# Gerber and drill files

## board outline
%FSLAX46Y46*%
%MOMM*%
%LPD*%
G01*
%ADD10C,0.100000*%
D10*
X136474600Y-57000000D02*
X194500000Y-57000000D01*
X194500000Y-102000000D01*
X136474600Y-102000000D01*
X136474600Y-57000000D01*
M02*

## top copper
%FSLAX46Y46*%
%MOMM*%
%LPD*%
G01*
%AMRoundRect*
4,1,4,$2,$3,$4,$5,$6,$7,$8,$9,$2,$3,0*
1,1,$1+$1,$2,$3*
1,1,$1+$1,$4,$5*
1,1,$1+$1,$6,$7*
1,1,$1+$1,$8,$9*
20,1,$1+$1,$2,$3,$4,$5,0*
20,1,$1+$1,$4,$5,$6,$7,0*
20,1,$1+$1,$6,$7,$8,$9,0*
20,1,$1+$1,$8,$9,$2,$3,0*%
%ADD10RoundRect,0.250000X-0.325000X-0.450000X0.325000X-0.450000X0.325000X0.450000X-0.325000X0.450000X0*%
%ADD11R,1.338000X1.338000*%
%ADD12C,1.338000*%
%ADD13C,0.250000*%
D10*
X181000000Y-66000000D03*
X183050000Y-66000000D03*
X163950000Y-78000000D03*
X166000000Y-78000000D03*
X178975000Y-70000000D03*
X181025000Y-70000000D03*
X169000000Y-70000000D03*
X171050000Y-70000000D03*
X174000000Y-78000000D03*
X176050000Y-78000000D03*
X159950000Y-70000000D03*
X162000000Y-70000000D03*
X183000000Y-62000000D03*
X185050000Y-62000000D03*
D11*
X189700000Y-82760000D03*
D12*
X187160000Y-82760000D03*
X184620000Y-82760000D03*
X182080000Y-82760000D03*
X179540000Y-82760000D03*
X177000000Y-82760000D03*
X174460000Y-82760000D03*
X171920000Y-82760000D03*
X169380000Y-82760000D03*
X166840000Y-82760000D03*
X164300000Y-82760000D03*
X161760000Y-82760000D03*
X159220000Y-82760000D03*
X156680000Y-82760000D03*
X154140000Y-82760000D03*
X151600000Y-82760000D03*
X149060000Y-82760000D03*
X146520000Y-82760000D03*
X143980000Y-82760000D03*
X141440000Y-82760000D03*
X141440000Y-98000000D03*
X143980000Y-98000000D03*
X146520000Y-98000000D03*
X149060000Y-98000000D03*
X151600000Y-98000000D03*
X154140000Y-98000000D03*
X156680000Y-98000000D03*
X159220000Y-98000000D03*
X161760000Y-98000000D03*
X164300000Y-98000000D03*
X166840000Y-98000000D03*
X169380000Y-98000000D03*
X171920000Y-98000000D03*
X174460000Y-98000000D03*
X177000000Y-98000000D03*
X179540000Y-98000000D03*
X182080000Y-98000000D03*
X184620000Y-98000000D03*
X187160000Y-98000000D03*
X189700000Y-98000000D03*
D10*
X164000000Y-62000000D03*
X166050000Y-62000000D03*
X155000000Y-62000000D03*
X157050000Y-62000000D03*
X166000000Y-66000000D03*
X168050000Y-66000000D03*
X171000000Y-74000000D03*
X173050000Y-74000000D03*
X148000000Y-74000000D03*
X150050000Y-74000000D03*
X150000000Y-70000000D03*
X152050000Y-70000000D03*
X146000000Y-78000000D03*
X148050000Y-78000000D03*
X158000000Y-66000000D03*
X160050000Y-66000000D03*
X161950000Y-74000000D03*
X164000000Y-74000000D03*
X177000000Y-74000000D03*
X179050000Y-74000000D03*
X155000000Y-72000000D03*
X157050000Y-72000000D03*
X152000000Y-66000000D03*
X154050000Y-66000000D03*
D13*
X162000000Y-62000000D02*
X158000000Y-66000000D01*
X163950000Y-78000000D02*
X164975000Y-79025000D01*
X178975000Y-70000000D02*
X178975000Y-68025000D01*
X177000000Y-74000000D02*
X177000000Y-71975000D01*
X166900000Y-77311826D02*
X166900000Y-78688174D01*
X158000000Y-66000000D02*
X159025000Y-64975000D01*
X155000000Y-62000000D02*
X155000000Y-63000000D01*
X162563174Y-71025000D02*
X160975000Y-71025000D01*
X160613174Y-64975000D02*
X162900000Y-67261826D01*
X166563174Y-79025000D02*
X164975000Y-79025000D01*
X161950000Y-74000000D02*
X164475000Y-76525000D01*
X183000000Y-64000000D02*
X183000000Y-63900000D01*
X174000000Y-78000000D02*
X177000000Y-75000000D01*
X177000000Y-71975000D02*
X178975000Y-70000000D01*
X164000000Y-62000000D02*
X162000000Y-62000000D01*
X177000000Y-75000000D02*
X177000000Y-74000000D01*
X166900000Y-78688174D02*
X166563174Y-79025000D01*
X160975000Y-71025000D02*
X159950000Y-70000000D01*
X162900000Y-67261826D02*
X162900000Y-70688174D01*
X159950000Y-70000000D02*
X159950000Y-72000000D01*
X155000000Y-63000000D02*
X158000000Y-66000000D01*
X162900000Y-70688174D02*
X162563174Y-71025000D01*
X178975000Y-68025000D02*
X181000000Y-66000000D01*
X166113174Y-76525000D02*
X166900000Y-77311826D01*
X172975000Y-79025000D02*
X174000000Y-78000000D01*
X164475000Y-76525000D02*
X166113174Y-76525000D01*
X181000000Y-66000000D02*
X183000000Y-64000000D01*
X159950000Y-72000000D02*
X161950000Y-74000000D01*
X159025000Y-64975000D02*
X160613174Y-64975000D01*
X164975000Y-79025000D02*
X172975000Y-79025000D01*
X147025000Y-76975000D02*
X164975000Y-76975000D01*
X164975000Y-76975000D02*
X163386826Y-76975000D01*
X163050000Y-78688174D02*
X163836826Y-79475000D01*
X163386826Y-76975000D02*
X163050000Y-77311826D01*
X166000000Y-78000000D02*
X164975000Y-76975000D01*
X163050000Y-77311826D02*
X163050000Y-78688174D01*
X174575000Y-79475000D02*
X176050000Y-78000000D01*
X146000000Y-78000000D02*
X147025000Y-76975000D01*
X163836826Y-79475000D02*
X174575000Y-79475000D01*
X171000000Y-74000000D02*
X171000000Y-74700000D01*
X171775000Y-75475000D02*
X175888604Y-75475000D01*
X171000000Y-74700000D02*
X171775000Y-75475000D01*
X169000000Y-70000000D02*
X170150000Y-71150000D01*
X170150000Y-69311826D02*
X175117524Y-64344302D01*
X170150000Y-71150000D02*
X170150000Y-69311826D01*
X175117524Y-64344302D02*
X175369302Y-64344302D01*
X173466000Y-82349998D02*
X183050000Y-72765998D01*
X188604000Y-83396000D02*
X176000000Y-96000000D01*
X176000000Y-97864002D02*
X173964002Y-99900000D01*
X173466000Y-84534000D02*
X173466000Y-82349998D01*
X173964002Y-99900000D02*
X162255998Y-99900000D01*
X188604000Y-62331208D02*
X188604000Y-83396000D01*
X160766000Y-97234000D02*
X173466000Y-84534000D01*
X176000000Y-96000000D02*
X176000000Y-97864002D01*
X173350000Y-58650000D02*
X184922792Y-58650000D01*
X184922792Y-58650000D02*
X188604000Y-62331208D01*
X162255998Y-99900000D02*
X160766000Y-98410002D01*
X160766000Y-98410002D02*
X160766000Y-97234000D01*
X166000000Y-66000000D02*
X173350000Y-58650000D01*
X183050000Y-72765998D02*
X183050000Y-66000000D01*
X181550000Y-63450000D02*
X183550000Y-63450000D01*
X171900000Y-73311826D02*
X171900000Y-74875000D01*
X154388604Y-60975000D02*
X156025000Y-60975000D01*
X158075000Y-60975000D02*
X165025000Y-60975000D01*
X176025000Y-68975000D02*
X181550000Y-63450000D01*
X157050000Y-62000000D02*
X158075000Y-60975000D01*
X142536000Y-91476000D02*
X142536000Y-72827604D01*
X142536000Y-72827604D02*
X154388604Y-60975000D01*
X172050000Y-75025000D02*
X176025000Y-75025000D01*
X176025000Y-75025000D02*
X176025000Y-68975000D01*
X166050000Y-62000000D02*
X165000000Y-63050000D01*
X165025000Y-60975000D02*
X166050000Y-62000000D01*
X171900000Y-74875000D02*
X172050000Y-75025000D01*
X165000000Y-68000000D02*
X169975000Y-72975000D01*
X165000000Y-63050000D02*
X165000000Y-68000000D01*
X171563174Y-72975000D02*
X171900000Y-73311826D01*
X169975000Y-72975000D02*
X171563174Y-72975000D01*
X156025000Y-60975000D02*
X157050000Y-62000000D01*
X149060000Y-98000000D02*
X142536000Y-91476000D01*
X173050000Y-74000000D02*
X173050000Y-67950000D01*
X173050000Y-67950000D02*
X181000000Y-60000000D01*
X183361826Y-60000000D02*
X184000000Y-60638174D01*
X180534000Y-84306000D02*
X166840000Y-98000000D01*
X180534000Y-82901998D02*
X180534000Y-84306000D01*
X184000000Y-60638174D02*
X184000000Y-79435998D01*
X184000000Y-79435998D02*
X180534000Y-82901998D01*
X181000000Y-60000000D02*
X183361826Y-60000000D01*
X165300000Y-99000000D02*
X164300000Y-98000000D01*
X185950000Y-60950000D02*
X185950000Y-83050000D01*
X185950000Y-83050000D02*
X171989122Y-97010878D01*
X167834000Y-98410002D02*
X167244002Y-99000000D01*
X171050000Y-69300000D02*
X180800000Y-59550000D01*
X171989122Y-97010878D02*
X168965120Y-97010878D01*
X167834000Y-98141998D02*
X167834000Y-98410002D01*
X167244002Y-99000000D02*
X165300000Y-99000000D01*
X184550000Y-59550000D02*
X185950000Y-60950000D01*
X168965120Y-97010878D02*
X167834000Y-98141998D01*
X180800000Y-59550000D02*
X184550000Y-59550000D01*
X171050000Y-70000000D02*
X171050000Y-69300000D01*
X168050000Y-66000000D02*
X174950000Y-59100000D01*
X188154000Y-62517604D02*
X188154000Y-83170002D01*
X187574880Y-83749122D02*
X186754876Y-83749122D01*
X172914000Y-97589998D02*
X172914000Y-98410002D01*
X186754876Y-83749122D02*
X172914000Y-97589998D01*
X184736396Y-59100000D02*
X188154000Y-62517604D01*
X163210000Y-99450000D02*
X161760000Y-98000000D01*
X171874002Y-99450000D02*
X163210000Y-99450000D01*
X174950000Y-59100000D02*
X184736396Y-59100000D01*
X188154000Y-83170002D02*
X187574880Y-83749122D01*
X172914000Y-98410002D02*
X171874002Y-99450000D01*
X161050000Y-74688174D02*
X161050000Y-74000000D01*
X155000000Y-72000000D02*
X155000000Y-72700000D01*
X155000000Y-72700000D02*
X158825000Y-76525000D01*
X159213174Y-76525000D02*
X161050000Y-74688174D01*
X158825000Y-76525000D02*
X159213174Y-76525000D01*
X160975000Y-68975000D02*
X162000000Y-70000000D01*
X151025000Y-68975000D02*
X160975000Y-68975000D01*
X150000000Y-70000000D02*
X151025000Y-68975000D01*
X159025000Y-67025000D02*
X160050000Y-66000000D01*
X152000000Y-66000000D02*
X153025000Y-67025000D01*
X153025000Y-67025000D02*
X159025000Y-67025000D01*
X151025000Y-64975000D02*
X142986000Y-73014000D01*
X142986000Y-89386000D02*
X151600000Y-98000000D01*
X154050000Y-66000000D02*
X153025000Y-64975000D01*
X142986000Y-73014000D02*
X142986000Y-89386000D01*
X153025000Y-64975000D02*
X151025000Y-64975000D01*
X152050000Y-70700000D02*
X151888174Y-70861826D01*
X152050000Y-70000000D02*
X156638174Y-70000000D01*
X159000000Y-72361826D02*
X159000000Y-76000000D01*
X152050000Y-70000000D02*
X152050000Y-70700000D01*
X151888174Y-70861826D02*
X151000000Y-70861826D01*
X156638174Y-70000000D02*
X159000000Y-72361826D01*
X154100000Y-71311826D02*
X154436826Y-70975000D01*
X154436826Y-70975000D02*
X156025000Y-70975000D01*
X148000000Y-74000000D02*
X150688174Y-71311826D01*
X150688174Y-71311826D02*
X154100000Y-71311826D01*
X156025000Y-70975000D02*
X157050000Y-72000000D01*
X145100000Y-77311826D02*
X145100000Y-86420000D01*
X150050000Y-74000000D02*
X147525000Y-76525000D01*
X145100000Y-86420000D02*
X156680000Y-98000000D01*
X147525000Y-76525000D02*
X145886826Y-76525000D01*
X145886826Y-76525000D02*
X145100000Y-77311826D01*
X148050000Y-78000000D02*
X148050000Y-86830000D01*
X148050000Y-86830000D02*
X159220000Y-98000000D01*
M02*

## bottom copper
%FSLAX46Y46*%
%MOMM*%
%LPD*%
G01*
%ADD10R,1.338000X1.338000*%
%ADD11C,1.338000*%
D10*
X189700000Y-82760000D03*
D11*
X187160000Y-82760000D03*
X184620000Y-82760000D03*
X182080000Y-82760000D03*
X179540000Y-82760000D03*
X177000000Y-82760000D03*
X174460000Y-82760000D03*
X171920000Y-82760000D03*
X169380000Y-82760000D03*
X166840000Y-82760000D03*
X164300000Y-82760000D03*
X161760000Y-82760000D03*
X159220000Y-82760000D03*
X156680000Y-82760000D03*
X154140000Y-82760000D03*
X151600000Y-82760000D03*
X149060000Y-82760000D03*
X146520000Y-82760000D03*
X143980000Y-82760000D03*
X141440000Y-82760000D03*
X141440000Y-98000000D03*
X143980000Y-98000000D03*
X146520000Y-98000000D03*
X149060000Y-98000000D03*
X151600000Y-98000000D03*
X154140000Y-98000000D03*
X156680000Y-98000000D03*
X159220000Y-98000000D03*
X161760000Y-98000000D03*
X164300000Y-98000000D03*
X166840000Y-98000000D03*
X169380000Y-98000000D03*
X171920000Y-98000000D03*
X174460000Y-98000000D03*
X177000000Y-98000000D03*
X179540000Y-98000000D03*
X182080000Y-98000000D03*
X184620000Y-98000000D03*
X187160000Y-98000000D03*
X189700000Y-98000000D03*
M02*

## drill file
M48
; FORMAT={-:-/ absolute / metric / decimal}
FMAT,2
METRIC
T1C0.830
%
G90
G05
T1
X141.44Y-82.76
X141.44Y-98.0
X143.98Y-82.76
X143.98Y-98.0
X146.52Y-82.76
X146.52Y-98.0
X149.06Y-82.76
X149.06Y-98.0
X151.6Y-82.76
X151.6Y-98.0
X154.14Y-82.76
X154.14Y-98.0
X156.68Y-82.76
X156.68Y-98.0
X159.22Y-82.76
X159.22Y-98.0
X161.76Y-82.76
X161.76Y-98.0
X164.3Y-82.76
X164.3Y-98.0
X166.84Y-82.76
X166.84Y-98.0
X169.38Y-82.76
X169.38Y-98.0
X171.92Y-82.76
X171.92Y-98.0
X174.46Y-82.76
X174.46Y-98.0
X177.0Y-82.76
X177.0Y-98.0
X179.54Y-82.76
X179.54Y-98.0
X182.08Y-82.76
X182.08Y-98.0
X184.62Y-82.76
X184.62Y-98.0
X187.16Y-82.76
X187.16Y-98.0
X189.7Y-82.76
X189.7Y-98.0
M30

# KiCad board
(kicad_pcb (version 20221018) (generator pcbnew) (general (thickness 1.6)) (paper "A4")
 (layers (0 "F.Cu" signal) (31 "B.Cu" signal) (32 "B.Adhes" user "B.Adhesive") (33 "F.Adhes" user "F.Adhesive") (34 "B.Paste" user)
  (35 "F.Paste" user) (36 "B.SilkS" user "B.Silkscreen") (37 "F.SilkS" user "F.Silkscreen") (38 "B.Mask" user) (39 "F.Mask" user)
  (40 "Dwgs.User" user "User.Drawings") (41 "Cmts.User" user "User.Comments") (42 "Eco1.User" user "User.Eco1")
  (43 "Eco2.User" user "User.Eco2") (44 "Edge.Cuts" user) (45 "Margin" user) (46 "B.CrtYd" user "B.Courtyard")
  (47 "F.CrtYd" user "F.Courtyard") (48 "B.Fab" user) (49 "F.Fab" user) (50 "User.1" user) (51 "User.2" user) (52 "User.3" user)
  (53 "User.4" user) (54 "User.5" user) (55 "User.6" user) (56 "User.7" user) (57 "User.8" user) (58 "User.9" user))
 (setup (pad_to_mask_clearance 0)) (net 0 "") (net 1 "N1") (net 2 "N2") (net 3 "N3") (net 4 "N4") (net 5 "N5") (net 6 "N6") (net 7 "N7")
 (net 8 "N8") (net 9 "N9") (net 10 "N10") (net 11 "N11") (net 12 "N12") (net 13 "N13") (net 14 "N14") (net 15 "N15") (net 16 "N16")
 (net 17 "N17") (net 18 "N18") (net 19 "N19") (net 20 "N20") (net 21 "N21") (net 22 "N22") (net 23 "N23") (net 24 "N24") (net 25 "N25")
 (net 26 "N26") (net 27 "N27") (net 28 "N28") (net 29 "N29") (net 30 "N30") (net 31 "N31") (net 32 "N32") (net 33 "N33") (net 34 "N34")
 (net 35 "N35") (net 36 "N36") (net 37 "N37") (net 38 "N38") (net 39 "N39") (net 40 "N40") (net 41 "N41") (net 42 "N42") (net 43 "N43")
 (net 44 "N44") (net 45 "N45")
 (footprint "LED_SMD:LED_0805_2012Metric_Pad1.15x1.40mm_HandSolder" (layer "F.Cu") (at 182.025 66)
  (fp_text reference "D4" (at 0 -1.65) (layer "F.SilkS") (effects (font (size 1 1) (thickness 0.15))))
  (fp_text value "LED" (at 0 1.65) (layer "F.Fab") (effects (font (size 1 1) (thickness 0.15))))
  (pad "1" smd roundrect (at -1.025 0) (size 1.15 1.4) (layers "F.Cu" "F.Paste" "F.Mask") (roundrect_rratio 0.217391) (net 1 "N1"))
  (pad "2" smd roundrect (at 1.025 0) (size 1.15 1.4) (layers "F.Cu" "F.Paste" "F.Mask") (roundrect_rratio 0.217391) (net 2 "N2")))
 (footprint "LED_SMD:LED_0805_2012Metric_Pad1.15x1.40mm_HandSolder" (layer "F.Cu") (at 164.975 78)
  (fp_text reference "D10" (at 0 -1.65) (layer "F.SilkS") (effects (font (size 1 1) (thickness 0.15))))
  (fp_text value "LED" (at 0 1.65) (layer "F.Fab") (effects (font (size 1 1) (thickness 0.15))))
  (pad "1" smd roundrect (at -1.025 0) (size 1.15 1.4) (layers "F.Cu" "F.Paste" "F.Mask") (roundrect_rratio 0.217391) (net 1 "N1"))
  (pad "2" smd roundrect (at 1.025 0) (size 1.15 1.4) (layers "F.Cu" "F.Paste" "F.Mask") (roundrect_rratio 0.217391) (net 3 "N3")))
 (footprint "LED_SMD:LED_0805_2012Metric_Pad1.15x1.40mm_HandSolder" (layer "F.Cu") (at 180 70)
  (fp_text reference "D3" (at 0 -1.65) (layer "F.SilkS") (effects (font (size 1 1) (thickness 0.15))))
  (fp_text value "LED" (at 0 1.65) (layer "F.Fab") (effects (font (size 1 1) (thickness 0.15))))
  (pad "1" smd roundrect (at -1.025 0) (size 1.15 1.4) (layers "F.Cu" "F.Paste" "F.Mask") (roundrect_rratio 0.217391) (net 1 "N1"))
  (pad "2" smd roundrect (at 1.025 0) (size 1.15 1.4) (layers "F.Cu" "F.Paste" "F.Mask") (roundrect_rratio 0.217391) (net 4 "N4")))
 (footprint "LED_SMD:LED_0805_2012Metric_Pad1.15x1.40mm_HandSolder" (layer "F.Cu") (at 170.025 70)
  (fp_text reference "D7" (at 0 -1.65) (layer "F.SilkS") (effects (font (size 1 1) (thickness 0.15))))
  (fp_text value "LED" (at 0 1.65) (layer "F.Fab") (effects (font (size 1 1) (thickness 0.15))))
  (pad "1" smd roundrect (at -1.025 0) (size 1.15 1.4) (layers "F.Cu" "F.Paste" "F.Mask") (roundrect_rratio 0.217391) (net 4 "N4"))
  (pad "2" smd roundrect (at 1.025 0) (size 1.15 1.4) (layers "F.Cu" "F.Paste" "F.Mask") (roundrect_rratio 0.217391) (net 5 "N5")))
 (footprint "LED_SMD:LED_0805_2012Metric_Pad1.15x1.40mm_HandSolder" (layer "F.Cu") (at 175.025 78)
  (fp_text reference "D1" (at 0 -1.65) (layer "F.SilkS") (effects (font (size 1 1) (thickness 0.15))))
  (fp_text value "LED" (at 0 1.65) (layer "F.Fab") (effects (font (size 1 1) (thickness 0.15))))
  (pad "1" smd roundrect (at -1.025 0) (size 1.15 1.4) (layers "F.Cu" "F.Paste" "F.Mask") (roundrect_rratio 0.217391) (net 1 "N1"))
  (pad "2" smd roundrect (at 1.025 0) (size 1.15 1.4) (layers "F.Cu" "F.Paste" "F.Mask") (roundrect_rratio 0.217391) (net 3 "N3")))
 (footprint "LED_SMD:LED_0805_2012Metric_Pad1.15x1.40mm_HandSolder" (layer "F.Cu") (at 160.975 70)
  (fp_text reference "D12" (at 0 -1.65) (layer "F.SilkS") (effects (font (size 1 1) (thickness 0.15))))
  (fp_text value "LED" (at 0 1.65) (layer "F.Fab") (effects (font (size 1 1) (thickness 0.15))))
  (pad "1" smd roundrect (at -1.025 0) (size 1.15 1.4) (layers "F.Cu" "F.Paste" "F.Mask") (roundrect_rratio 0.217391) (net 1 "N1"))
  (pad "2" smd roundrect (at 1.025 0) (size 1.15 1.4) (layers "F.Cu" "F.Paste" "F.Mask") (roundrect_rratio 0.217391) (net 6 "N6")))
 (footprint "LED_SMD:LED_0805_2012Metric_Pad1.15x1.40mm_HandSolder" (layer "F.Cu") (at 184.025 62)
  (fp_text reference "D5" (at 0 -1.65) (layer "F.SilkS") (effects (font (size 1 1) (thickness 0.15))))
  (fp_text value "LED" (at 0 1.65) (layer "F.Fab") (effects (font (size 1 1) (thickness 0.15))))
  (pad "1" smd roundrect (at -1.025 0) (size 1.15 1.4) (layers "F.Cu" "F.Paste" "F.Mask") (roundrect_rratio 0.217391) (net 1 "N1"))
  (pad "2" smd roundrect (at 1.025 0) (size 1.15 1.4) (layers "F.Cu" "F.Paste" "F.Mask") (roundrect_rratio 0.217391) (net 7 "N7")))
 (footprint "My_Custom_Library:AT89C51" (layer "F.Cu") (at 165.57 90.38 -90)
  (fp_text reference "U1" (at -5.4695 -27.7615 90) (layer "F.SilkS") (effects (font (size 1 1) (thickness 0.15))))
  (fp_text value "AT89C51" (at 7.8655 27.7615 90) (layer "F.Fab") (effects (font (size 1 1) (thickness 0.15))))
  (pad "1" thru_hole rect (at -7.62 -24.13 270) (size 1.338 1.338) (drill 0.83) (layers "*.Cu" "*.Mask") (solder_mask_margin 0.102))
  (pad "2" thru_hole circle (at -7.62 -21.59 270) (size 1.338 1.338) (drill 0.83) (layers "*.Cu" "*.Mask") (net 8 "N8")
   (solder_mask_margin 0.102))
  (pad "3" thru_hole circle (at -7.62 -19.05 270) (size 1.338 1.338) (drill 0.83) (layers "*.Cu" "*.Mask") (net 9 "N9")
   (solder_mask_margin 0.102))
  (pad "4" thru_hole circle (at -7.62 -16.51 270) (size 1.338 1.338) (drill 0.83) (layers "*.Cu" "*.Mask") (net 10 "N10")
   (solder_mask_margin 0.102))
  (pad "5" thru_hole circle (at -7.62 -13.97 270) (size 1.338 1.338) (drill 0.83) (layers "*.Cu" "*.Mask") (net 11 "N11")
   (solder_mask_margin 0.102))
  (pad "6" thru_hole circle (at -7.62 -11.43 270) (size 1.338 1.338) (drill 0.83) (layers "*.Cu" "*.Mask") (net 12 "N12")
   (solder_mask_margin 0.102))
  (pad "7" thru_hole circle (at -7.62 -8.89 270) (size 1.338 1.338) (drill 0.83) (layers "*.Cu" "*.Mask") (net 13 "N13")
   (solder_mask_margin 0.102))
  (pad "8" thru_hole circle (at -7.62 -6.35 270) (size 1.338 1.338) (drill 0.83) (layers "*.Cu" "*.Mask") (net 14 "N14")
   (solder_mask_margin 0.102))
  (pad "9" thru_hole circle (at -7.62 -3.81 270) (size 1.338 1.338) (drill 0.83) (layers "*.Cu" "*.Mask") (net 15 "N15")
   (solder_mask_margin 0.102))
  (pad "10" thru_hole circle (at -7.62 -1.27 270) (size 1.338 1.338) (drill 0.83) (layers "*.Cu" "*.Mask") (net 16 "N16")
   (solder_mask_margin 0.102))
  (pad "11" thru_hole circle (at -7.62 1.27 270) (size 1.338 1.338) (drill 0.83) (layers "*.Cu" "*.Mask") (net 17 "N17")
   (solder_mask_margin 0.102))
  (pad "12" thru_hole circle (at -7.62 3.81 270) (size 1.338 1.338) (drill 0.83) (layers "*.Cu" "*.Mask") (solder_mask_margin 0.102))
  (pad "13" thru_hole circle (at -7.62 6.35 270) (size 1.338 1.338) (drill 0.83) (layers "*.Cu" "*.Mask") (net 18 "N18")
   (solder_mask_margin 0.102))
  (pad "14" thru_hole circle (at -7.62 8.89 270) (size 1.338 1.338) (drill 0.83) (layers "*.Cu" "*.Mask") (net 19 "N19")
   (solder_mask_margin 0.102))
  (pad "15" thru_hole circle (at -7.62 11.43 270) (size 1.338 1.338) (drill 0.83) (layers "*.Cu" "*.Mask") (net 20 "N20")
   (solder_mask_margin 0.102))
  (pad "16" thru_hole circle (at -7.62 13.97 270) (size 1.338 1.338) (drill 0.83) (layers "*.Cu" "*.Mask") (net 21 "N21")
   (solder_mask_margin 0.102))
  (pad "17" thru_hole circle (at -7.62 16.51 270) (size 1.338 1.338) (drill 0.83) (layers "*.Cu" "*.Mask") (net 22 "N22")
   (solder_mask_margin 0.102))
  (pad "18" thru_hole circle (at -7.62 19.05 270) (size 1.338 1.338) (drill 0.83) (layers "*.Cu" "*.Mask") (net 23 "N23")
   (solder_mask_margin 0.102))
  (pad "19" thru_hole circle (at -7.62 21.59 270) (size 1.338 1.338) (drill 0.83) (layers "*.Cu" "*.Mask") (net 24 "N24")
   (solder_mask_margin 0.102))
  (pad "20" thru_hole circle (at -7.62 24.13 270) (size 1.338 1.338) (drill 0.83) (layers "*.Cu" "*.Mask") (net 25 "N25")
   (solder_mask_margin 0.102))
  (pad "21" thru_hole circle (at 7.62 24.13 270) (size 1.338 1.338) (drill 0.83) (layers "*.Cu" "*.Mask") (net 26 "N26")
   (solder_mask_margin 0.102))
  (pad "22" thru_hole circle (at 7.62 21.59 270) (size 1.338 1.338) (drill 0.83) (layers "*.Cu" "*.Mask") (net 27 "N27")
   (solder_mask_margin 0.102))
  (pad "23" thru_hole circle (at 7.62 19.05 270) (size 1.338 1.338) (drill 0.83) (layers "*.Cu" "*.Mask") (solder_mask_margin 0.102))
  (pad "24" thru_hole circle (at 7.62 16.51 270) (size 1.338 1.338) (drill 0.83) (layers "*.Cu" "*.Mask") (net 7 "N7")
   (solder_mask_margin 0.102))
  (pad "25" thru_hole circle (at 7.62 13.97 270) (size 1.338 1.338) (drill 0.83) (layers "*.Cu" "*.Mask") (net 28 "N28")
   (solder_mask_margin 0.102))
  (pad "26" thru_hole circle (at 7.62 11.43 270) (size 1.338 1.338) (drill 0.83) (layers "*.Cu" "*.Mask") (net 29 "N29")
   (solder_mask_margin 0.102))
  (pad "27" thru_hole circle (at 7.62 8.89 270) (size 1.338 1.338) (drill 0.83) (layers "*.Cu" "*.Mask") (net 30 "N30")
   (solder_mask_margin 0.102))
  (pad "28" thru_hole circle (at 7.62 6.35 270) (size 1.338 1.338) (drill 0.83) (layers "*.Cu" "*.Mask") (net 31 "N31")
   (solder_mask_margin 0.102))
  (pad "29" thru_hole circle (at 7.62 3.81 270) (size 1.338 1.338) (drill 0.83) (layers "*.Cu" "*.Mask") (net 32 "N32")
   (solder_mask_margin 0.102))
  (pad "30" thru_hole circle (at 7.62 1.27 270) (size 1.338 1.338) (drill 0.83) (layers "*.Cu" "*.Mask") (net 5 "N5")
   (solder_mask_margin 0.102))
  (pad "31" thru_hole circle (at 7.62 -1.27 270) (size 1.338 1.338) (drill 0.83) (layers "*.Cu" "*.Mask") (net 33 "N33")
   (solder_mask_margin 0.102))
  (pad "32" thru_hole circle (at 7.62 -3.81 270) (size 1.338 1.338) (drill 0.83) (layers "*.Cu" "*.Mask") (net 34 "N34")
   (solder_mask_margin 0.102))
  (pad "33" thru_hole circle (at 7.62 -6.35 270) (size 1.338 1.338) (drill 0.83) (layers "*.Cu" "*.Mask") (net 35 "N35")
   (solder_mask_margin 0.102))
  (pad "34" thru_hole circle (at 7.62 -8.89 270) (size 1.338 1.338) (drill 0.83) (layers "*.Cu" "*.Mask") (solder_mask_margin 0.102))
  (pad "35" thru_hole circle (at 7.62 -11.43 270) (size 1.338 1.338) (drill 0.83) (layers "*.Cu" "*.Mask") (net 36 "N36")
   (solder_mask_margin 0.102))
  (pad "36" thru_hole circle (at 7.62 -13.97 270) (size 1.338 1.338) (drill 0.83) (layers "*.Cu" "*.Mask") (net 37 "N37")
   (solder_mask_margin 0.102))
  (pad "37" thru_hole circle (at 7.62 -16.51 270) (size 1.338 1.338) (drill 0.83) (layers "*.Cu" "*.Mask") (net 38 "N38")
   (solder_mask_margin 0.102))
  (pad "38" thru_hole circle (at 7.62 -19.05 270) (size 1.338 1.338) (drill 0.83) (layers "*.Cu" "*.Mask") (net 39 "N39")
   (solder_mask_margin 0.102))
  (pad "39" thru_hole circle (at 7.62 -21.59 270) (size 1.338 1.338) (drill 0.83) (layers "*.Cu" "*.Mask") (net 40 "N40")
   (solder_mask_margin 0.102))
  (pad "40" thru_hole circle (at 7.62 -24.13 270) (size 1.338 1.338) (drill 0.83) (layers "*.Cu" "*.Mask") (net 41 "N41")
   (solder_mask_margin 0.102)))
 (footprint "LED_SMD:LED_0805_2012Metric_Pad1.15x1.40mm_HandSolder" (layer "F.Cu") (at 165.025 62)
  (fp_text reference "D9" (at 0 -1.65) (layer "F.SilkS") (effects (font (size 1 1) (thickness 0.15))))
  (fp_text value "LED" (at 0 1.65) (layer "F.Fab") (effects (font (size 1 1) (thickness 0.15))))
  (pad "1" smd roundrect (at -1.025 0) (size 1.15 1.4) (layers "F.Cu" "F.Paste" "F.Mask") (roundrect_rratio 0.217391) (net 1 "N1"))
  (pad "2" smd roundrect (at 1.025 0) (size 1.15 1.4) (layers "F.Cu" "F.Paste" "F.Mask") (roundrect_rratio 0.217391) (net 7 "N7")))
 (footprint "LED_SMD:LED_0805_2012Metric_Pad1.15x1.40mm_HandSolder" (layer "F.Cu") (at 156.025 62)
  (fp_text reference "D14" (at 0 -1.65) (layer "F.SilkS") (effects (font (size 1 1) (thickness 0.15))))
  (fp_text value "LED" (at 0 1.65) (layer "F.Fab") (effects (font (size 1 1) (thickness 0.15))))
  (pad "1" smd roundrect (at -1.025 0) (size 1.15 1.4) (layers "F.Cu" "F.Paste" "F.Mask") (roundrect_rratio 0.217391) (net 1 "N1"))
  (pad "2" smd roundrect (at 1.025 0) (size 1.15 1.4) (layers "F.Cu" "F.Paste" "F.Mask") (roundrect_rratio 0.217391) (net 7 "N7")))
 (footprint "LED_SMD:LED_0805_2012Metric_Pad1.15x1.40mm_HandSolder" (layer "F.Cu") (at 167.025 66)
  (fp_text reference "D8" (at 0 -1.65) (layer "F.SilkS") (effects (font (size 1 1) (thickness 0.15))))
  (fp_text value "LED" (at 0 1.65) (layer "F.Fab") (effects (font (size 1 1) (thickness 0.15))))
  (pad "1" smd roundrect (at -1.025 0) (size 1.15 1.4) (layers "F.Cu" "F.Paste" "F.Mask") (roundrect_rratio 0.217391) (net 2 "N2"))
  (pad "2" smd roundrect (at 1.025 0) (size 1.15 1.4) (layers "F.Cu" "F.Paste" "F.Mask") (roundrect_rratio 0.217391) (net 32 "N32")))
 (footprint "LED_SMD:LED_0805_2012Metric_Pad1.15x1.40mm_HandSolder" (layer "F.Cu") (at 172.025 74)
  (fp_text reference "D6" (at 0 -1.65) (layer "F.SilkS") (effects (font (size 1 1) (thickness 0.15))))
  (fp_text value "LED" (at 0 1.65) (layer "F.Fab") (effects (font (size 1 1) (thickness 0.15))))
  (pad "1" smd roundrect (at -1.025 0) (size 1.15 1.4) (layers "F.Cu" "F.Paste" "F.Mask") (roundrect_rratio 0.217391) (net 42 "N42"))
  (pad "2" smd roundrect (at 1.025 0) (size 1.15 1.4) (layers "F.Cu" "F.Paste" "F.Mask") (roundrect_rratio 0.217391) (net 33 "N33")))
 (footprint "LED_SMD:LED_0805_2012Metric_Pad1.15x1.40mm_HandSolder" (layer "F.Cu") (at 149.025 74)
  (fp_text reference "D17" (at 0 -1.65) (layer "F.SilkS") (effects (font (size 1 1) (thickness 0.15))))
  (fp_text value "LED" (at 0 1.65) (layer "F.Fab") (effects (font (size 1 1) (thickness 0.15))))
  (pad "1" smd roundrect (at -1.025 0) (size 1.15 1.4) (layers "F.Cu" "F.Paste" "F.Mask") (roundrect_rratio 0.217391) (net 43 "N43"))
  (pad "2" smd roundrect (at 1.025 0) (size 1.15 1.4) (layers "F.Cu" "F.Paste" "F.Mask") (roundrect_rratio 0.217391) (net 30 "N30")))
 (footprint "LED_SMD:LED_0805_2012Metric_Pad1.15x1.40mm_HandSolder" (layer "F.Cu") (at 151.025 70)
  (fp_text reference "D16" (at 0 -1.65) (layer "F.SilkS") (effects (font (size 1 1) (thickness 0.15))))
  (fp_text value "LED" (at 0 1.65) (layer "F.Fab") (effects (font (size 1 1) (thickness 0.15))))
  (pad "1" smd roundrect (at -1.025 0) (size 1.15 1.4) (layers "F.Cu" "F.Paste" "F.Mask") (roundrect_rratio 0.217391) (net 6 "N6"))
  (pad "2" smd roundrect (at 1.025 0) (size 1.15 1.4) (layers "F.Cu" "F.Paste" "F.Mask") (roundrect_rratio 0.217391) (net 29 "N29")))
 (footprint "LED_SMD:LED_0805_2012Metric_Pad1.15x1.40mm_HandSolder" (layer "F.Cu") (at 147.025 78)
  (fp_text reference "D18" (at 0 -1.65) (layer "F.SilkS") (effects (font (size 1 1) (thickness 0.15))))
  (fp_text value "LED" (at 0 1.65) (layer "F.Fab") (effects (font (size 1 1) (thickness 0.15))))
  (pad "1" smd roundrect (at -1.025 0) (size 1.15 1.4) (layers "F.Cu" "F.Paste" "F.Mask") (roundrect_rratio 0.217391) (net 3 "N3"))
  (pad "2" smd roundrect (at 1.025 0) (size 1.15 1.4) (layers "F.Cu" "F.Paste" "F.Mask") (roundrect_rratio 0.217391) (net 31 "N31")))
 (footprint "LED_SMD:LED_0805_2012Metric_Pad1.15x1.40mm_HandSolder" (layer "F.Cu") (at 159.025 66)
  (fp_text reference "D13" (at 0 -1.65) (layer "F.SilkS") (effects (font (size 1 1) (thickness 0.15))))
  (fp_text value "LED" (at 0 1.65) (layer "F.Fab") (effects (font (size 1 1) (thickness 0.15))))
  (pad "1" smd roundrect (at -1.025 0) (size 1.15 1.4) (layers "F.Cu" "F.Paste" "F.Mask") (roundrect_rratio 0.217391) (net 1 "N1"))
  (pad "2" smd roundrect (at 1.025 0) (size 1.15 1.4) (layers "F.Cu" "F.Paste" "F.Mask") (roundrect_rratio 0.217391) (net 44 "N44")))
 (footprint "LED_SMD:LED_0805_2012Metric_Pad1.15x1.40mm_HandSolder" (layer "F.Cu") (at 162.975 74)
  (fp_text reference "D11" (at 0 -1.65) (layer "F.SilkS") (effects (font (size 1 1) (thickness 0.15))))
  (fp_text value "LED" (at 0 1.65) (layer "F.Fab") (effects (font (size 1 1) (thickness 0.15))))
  (pad "1" smd roundrect (at -1.025 0) (size 1.15 1.4) (layers "F.Cu" "F.Paste" "F.Mask") (roundrect_rratio 0.217391) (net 1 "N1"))
  (pad "2" smd roundrect (at 1.025 0) (size 1.15 1.4) (layers "F.Cu" "F.Paste" "F.Mask") (roundrect_rratio 0.217391) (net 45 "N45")))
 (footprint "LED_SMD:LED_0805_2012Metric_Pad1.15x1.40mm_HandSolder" (layer "F.Cu") (at 178.025 74)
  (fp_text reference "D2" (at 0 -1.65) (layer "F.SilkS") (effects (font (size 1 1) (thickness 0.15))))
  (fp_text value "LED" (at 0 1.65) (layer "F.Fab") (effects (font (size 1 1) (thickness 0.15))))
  (pad "1" smd roundrect (at -1.025 0) (size 1.15 1.4) (layers "F.Cu" "F.Paste" "F.Mask") (roundrect_rratio 0.217391) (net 1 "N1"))
  (pad "2" smd roundrect (at 1.025 0) (size 1.15 1.4) (layers "F.Cu" "F.Paste" "F.Mask") (roundrect_rratio 0.217391) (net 42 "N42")))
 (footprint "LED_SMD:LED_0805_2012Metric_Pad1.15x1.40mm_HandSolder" (layer "F.Cu") (at 156.025 72)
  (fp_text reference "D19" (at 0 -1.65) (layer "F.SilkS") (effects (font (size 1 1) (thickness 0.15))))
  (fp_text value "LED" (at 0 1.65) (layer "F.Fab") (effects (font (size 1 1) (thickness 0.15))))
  (pad "1" smd roundrect (at -1.025 0) (size 1.15 1.4) (layers "F.Cu" "F.Paste" "F.Mask") (roundrect_rratio 0.217391) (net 45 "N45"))
  (pad "2" smd roundrect (at 1.025 0) (size 1.15 1.4) (layers "F.Cu" "F.Paste" "F.Mask") (roundrect_rratio 0.217391) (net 43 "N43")))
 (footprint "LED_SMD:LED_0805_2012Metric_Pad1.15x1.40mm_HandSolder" (layer "F.Cu") (at 153.025 66)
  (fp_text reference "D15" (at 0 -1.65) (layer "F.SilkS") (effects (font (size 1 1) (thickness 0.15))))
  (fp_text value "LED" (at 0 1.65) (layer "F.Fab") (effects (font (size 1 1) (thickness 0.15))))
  (pad "1" smd roundrect (at -1.025 0) (size 1.15 1.4) (layers "F.Cu" "F.Paste" "F.Mask") (roundrect_rratio 0.217391) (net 44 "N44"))
  (pad "2" smd roundrect (at 1.025 0) (size 1.15 1.4) (layers "F.Cu" "F.Paste" "F.Mask") (roundrect_rratio 0.217391) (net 28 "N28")))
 (gr_rect (start 136.4746 57) (end 194.5 102) (stroke (width 0.1) (type default)) (fill none) (layer "Edge.Cuts"))
 (segment (start 162 62) (end 158 66) (width 0.25) (layer "F.Cu") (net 1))
 (segment (start 163.95 78) (end 164.975 79.025) (width 0.25) (layer "F.Cu") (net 1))
 (segment (start 178.975 70) (end 178.975 68.025) (width 0.25) (layer "F.Cu") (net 1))
 (segment (start 177 74) (end 177 71.975) (width 0.25) (layer "F.Cu") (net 1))
 (segment (start 166.9 77.311826) (end 166.9 78.688174) (width 0.25) (layer "F.Cu") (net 1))
 (segment (start 158 66) (end 159.025 64.975) (width 0.25) (layer "F.Cu") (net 1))
 (segment (start 155 62) (end 155 63) (width 0.25) (layer "F.Cu") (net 1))
 (segment (start 162.563174 71.025) (end 160.975 71.025) (width 0.25) (layer "F.Cu") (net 1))
 (segment (start 160.613174 64.975) (end 162.9 67.261826) (width 0.25) (layer "F.Cu") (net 1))
 (segment (start 166.563174 79.025) (end 164.975 79.025) (width 0.25) (layer "F.Cu") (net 1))
 (segment (start 161.95 74) (end 164.475 76.525) (width 0.25) (layer "F.Cu") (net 1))
 (segment (start 183 64) (end 183 63.9) (width 0.25) (layer "F.Cu") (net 1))
 (segment (start 174 78) (end 177 75) (width 0.25) (layer "F.Cu") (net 1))
 (segment (start 177 71.975) (end 178.975 70) (width 0.25) (layer "F.Cu") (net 1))
 (segment (start 164 62) (end 162 62) (width 0.25) (layer "F.Cu") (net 1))
 (segment (start 177 75) (end 177 74) (width 0.25) (layer "F.Cu") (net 1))
 (segment (start 166.9 78.688174) (end 166.563174 79.025) (width 0.25) (layer "F.Cu") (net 1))
 (segment (start 160.975 71.025) (end 159.95 70) (width 0.25) (layer "F.Cu") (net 1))
 (segment (start 162.9 67.261826) (end 162.9 70.688174) (width 0.25) (layer "F.Cu") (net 1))
 (segment (start 159.95 70) (end 159.95 72) (width 0.25) (layer "F.Cu") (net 1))
 (segment (start 155 63) (end 158 66) (width 0.25) (layer "F.Cu") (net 1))
 (segment (start 162.9 70.688174) (end 162.563174 71.025) (width 0.25) (layer "F.Cu") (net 1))
 (segment (start 178.975 68.025) (end 181 66) (width 0.25) (layer "F.Cu") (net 1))
 (segment (start 166.113174 76.525) (end 166.9 77.311826) (width 0.25) (layer "F.Cu") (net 1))
 (segment (start 172.975 79.025) (end 174 78) (width 0.25) (layer "F.Cu") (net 1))
 (segment (start 164.475 76.525) (end 166.113174 76.525) (width 0.25) (layer "F.Cu") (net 1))
 (segment (start 181 66) (end 183 64) (width 0.25) (layer "F.Cu") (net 1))
 (segment (start 159.95 72) (end 161.95 74) (width 0.25) (layer "F.Cu") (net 1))
 (segment (start 159.025 64.975) (end 160.613174 64.975) (width 0.25) (layer "F.Cu") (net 1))
 (segment (start 164.975 79.025) (end 172.975 79.025) (width 0.25) (layer "F.Cu") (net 1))
 (segment (start 147.025 76.975) (end 164.975 76.975) (width 0.25) (layer "F.Cu") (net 3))
 (segment (start 164.975 76.975) (end 163.386826 76.975) (width 0.25) (layer "F.Cu") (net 3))
 (segment (start 163.05 78.688174) (end 163.836826 79.475) (width 0.25) (layer "F.Cu") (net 3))
 (segment (start 163.386826 76.975) (end 163.05 77.311826) (width 0.25) (layer "F.Cu") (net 3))
 (segment (start 166 78) (end 164.975 76.975) (width 0.25) (layer "F.Cu") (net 3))
 (segment (start 163.05 77.311826) (end 163.05 78.688174) (width 0.25) (layer "F.Cu") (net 3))
 (segment (start 174.575 79.475) (end 176.05 78) (width 0.25) (layer "F.Cu") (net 3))
 (segment (start 146 78) (end 147.025 76.975) (width 0.25) (layer "F.Cu") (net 3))
 (segment (start 163.836826 79.475) (end 174.575 79.475) (width 0.25) (layer "F.Cu") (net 3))
 (segment (start 171 74) (end 171 74.7) (width 0.25) (layer "F.Cu") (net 42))
 (segment (start 171.775 75.475) (end 175.888604 75.475) (width 0.25) (layer "F.Cu") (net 42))
 (segment (start 171 74.7) (end 171.775 75.475) (width 0.25) (layer "F.Cu") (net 42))
 (segment (start 169 70) (end 170.15 71.15) (width 0.25) (layer "F.Cu") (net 4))
 (segment (start 170.15 69.311826) (end 175.117524 64.344302) (width 0.25) (layer "F.Cu") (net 4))
 (segment (start 170.15 71.15) (end 170.15 69.311826) (width 0.25) (layer "F.Cu") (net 4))
 (segment (start 175.117524 64.344302) (end 175.369302 64.344302) (width 0.25) (layer "F.Cu") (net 4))
 (segment (start 173.466 82.349998) (end 183.05 72.765998) (width 0.25) (layer "F.Cu") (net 2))
 (segment (start 188.604 83.396) (end 176 96) (width 0.25) (layer "F.Cu") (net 2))
 (segment (start 176 97.864002) (end 173.964002 99.9) (width 0.25) (layer "F.Cu") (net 2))
 (segment (start 173.466 84.534) (end 173.466 82.349998) (width 0.25) (layer "F.Cu") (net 2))
 (segment (start 173.964002 99.9) (end 162.255998 99.9) (width 0.25) (layer "F.Cu") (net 2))
 (segment (start 188.604 62.331208) (end 188.604 83.396) (width 0.25) (layer "F.Cu") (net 2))
 (segment (start 160.766 97.234) (end 173.466 84.534) (width 0.25) (layer "F.Cu") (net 2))
 (segment (start 176 96) (end 176 97.864002) (width 0.25) (layer "F.Cu") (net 2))
 (segment (start 173.35 58.65) (end 184.922792 58.65) (width 0.25) (layer "F.Cu") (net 2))
 (segment (start 184.922792 58.65) (end 188.604 62.331208) (width 0.25) (layer "F.Cu") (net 2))
 (segment (start 162.255998 99.9) (end 160.766 98.410002) (width 0.25) (layer "F.Cu") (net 2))
 (segment (start 160.766 98.410002) (end 160.766 97.234) (width 0.25) (layer "F.Cu") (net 2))
 (segment (start 166 66) (end 173.35 58.65) (width 0.25) (layer "F.Cu") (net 2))
 (segment (start 183.05 72.765998) (end 183.05 66) (width 0.25) (layer "F.Cu") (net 2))
 (segment (start 181.55 63.45) (end 183.55 63.45) (width 0.25) (layer "F.Cu") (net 7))
 (segment (start 171.9 73.311826) (end 171.9 74.875) (width 0.25) (layer "F.Cu") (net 7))
 (segment (start 154.388604 60.975) (end 156.025 60.975) (width 0.25) (layer "F.Cu") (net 7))
 (segment (start 158.075 60.975) (end 165.025 60.975) (width 0.25) (layer "F.Cu") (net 7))
 (segment (start 176.025 68.975) (end 181.55 63.45) (width 0.25) (layer "F.Cu") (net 7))
 (segment (start 157.05 62) (end 158.075 60.975) (width 0.25) (layer "F.Cu") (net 7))
 (segment (start 142.536 91.476) (end 142.536 72.827604) (width 0.25) (layer "F.Cu") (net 7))
 (segment (start 142.536 72.827604) (end 154.388604 60.975) (width 0.25) (layer "F.Cu") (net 7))
 (segment (start 172.05 75.025) (end 176.025 75.025) (width 0.25) (layer "F.Cu") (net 7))
 (segment (start 176.025 75.025) (end 176.025 68.975) (width 0.25) (layer "F.Cu") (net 7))
 (segment (start 166.05 62) (end 165 63.05) (width 0.25) (layer "F.Cu") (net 7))
 (segment (start 165.025 60.975) (end 166.05 62) (width 0.25) (layer "F.Cu") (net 7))
 (segment (start 171.9 74.875) (end 172.05 75.025) (width 0.25) (layer "F.Cu") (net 7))
 (segment (start 165 68) (end 169.975 72.975) (width 0.25) (layer "F.Cu") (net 7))
 (segment (start 165 63.05) (end 165 68) (width 0.25) (layer "F.Cu") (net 7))
 (segment (start 171.563174 72.975) (end 171.9 73.311826) (width 0.25) (layer "F.Cu") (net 7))
 (segment (start 169.975 72.975) (end 171.563174 72.975) (width 0.25) (layer "F.Cu") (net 7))
 (segment (start 156.025 60.975) (end 157.05 62) (width 0.25) (layer "F.Cu") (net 7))
 (segment (start 149.06 98) (end 142.536 91.476) (width 0.25) (layer "F.Cu") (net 7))
 (segment (start 173.05 74) (end 173.05 67.95) (width 0.25) (layer "F.Cu") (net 33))
 (segment (start 173.05 67.95) (end 181 60) (width 0.25) (layer "F.Cu") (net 33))
 (segment (start 183.361826 60) (end 184 60.638174) (width 0.25) (layer "F.Cu") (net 33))
 (segment (start 180.534 84.306) (end 166.84 98) (width 0.25) (layer "F.Cu") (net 33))
 (segment (start 180.534 82.901998) (end 180.534 84.306) (width 0.25) (layer "F.Cu") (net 33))
 (segment (start 184 60.638174) (end 184 79.435998) (width 0.25) (layer "F.Cu") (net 33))
 (segment (start 184 79.435998) (end 180.534 82.901998) (width 0.25) (layer "F.Cu") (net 33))
 (segment (start 181 60) (end 183.361826 60) (width 0.25) (layer "F.Cu") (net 33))
 (segment (start 165.3 99) (end 164.3 98) (width 0.25) (layer "F.Cu") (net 5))
 (segment (start 185.95 60.95) (end 185.95 83.05) (width 0.25) (layer "F.Cu") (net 5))
 (segment (start 185.95 83.05) (end 171.989122 97.010878) (width 0.25) (layer "F.Cu") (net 5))
 (segment (start 167.834 98.410002) (end 167.244002 99) (width 0.25) (layer "F.Cu") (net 5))
 (segment (start 171.05 69.3) (end 180.8 59.55) (width 0.25) (layer "F.Cu") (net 5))
 (segment (start 171.989122 97.010878) (end 168.96512 97.010878) (width 0.25) (layer "F.Cu") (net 5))
 (segment (start 167.834 98.141998) (end 167.834 98.410002) (width 0.25) (layer "F.Cu") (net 5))
 (segment (start 167.244002 99) (end 165.3 99) (width 0.25) (layer "F.Cu") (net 5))
 (segment (start 184.55 59.55) (end 185.95 60.95) (width 0.25) (layer "F.Cu") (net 5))
 (segment (start 168.96512 97.010878) (end 167.834 98.141998) (width 0.25) (layer "F.Cu") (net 5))
 (segment (start 180.8 59.55) (end 184.55 59.55) (width 0.25) (layer "F.Cu") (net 5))
 (segment (start 171.05 70) (end 171.05 69.3) (width 0.25) (layer "F.Cu") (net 5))
 (segment (start 168.05 66) (end 174.95 59.1) (width 0.25) (layer "F.Cu") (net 32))
 (segment (start 188.154 62.517604) (end 188.154 83.170002) (width 0.25) (layer "F.Cu") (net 32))
 (segment (start 187.57488 83.749122) (end 186.754876 83.749122) (width 0.25) (layer "F.Cu") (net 32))
 (segment (start 172.914 97.589998) (end 172.914 98.410002) (width 0.25) (layer "F.Cu") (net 32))
 (segment (start 186.754876 83.749122) (end 172.914 97.589998) (width 0.25) (layer "F.Cu") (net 32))
 (segment (start 184.736396 59.1) (end 188.154 62.517604) (width 0.25) (layer "F.Cu") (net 32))
 (segment (start 163.21 99.45) (end 161.76 98) (width 0.25) (layer "F.Cu") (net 32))
 (segment (start 171.874002 99.45) (end 163.21 99.45) (width 0.25) (layer "F.Cu") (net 32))
 (segment (start 174.95 59.1) (end 184.736396 59.1) (width 0.25) (layer "F.Cu") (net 32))
 (segment (start 188.154 83.170002) (end 187.57488 83.749122) (width 0.25) (layer "F.Cu") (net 32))
 (segment (start 172.914 98.410002) (end 171.874002 99.45) (width 0.25) (layer "F.Cu") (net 32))
 (segment (start 161.05 74.688174) (end 161.05 74) (width 0.25) (layer "F.Cu") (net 45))
 (segment (start 155 72) (end 155 72.7) (width 0.25) (layer "F.Cu") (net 45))
 (segment (start 155 72.7) (end 158.825 76.525) (width 0.25) (layer "F.Cu") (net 45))
 (segment (start 159.213174 76.525) (end 161.05 74.688174) (width 0.25) (layer "F.Cu") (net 45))
 (segment (start 158.825 76.525) (end 159.213174 76.525) (width 0.25) (layer "F.Cu") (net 45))
 (segment (start 160.975 68.975) (end 162 70) (width 0.25) (layer "F.Cu") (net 6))
 (segment (start 151.025 68.975) (end 160.975 68.975) (width 0.25) (layer "F.Cu") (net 6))
 (segment (start 150 70) (end 151.025 68.975) (width 0.25) (layer "F.Cu") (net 6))
 (segment (start 159.025 67.025) (end 160.05 66) (width 0.25) (layer "F.Cu") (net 44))
 (segment (start 152 66) (end 153.025 67.025) (width 0.25) (layer "F.Cu") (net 44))
 (segment (start 153.025 67.025) (end 159.025 67.025) (width 0.25) (layer "F.Cu") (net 44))
 (segment (start 151.025 64.975) (end 142.986 73.014) (width 0.25) (layer "F.Cu") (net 28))
 (segment (start 142.986 89.386) (end 151.6 98) (width 0.25) (layer "F.Cu") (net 28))
 (segment (start 154.05 66) (end 153.025 64.975) (width 0.25) (layer "F.Cu") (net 28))
 (segment (start 142.986 73.014) (end 142.986 89.386) (width 0.25) (layer "F.Cu") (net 28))
 (segment (start 153.025 64.975) (end 151.025 64.975) (width 0.25) (layer "F.Cu") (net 28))
 (segment (start 152.05 70.7) (end 151.888174 70.861826) (width 0.25) (layer "F.Cu") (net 29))
 (segment (start 152.05 70) (end 156.638174 70) (width 0.25) (layer "F.Cu") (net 29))
 (segment (start 159 72.361826) (end 159 76) (width 0.25) (layer "F.Cu") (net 29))
 (segment (start 152.05 70) (end 152.05 70.7) (width 0.25) (layer "F.Cu") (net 29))
 (segment (start 151.888174 70.861826) (end 151 70.861826) (width 0.25) (layer "F.Cu") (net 29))
 (segment (start 156.638174 70) (end 159 72.361826) (width 0.25) (layer "F.Cu") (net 29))
 (segment (start 154.1 71.311826) (end 154.436826 70.975) (width 0.25) (layer "F.Cu") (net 43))
 (segment (start 154.436826 70.975) (end 156.025 70.975) (width 0.25) (layer "F.Cu") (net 43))
 (segment (start 148 74) (end 150.688174 71.311826) (width 0.25) (layer "F.Cu") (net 43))
 (segment (start 150.688174 71.311826) (end 154.1 71.311826) (width 0.25) (layer "F.Cu") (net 43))
 (segment (start 156.025 70.975) (end 157.05 72) (width 0.25) (layer "F.Cu") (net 43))
 (segment (start 145.1 77.311826) (end 145.1 86.42) (width 0.25) (layer "F.Cu") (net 30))
 (segment (start 150.05 74) (end 147.525 76.525) (width 0.25) (layer "F.Cu") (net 30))
 (segment (start 145.1 86.42) (end 156.68 98) (width 0.25) (layer "F.Cu") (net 30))
 (segment (start 147.525 76.525) (end 145.886826 76.525) (width 0.25) (layer "F.Cu") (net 30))
 (segment (start 145.886826 76.525) (end 145.1 77.311826) (width 0.25) (layer "F.Cu") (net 30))
 (segment (start 148.05 78) (end 148.05 86.83) (width 0.25) (layer "F.Cu") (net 31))
 (segment (start 148.05 86.83) (end 159.22 98) (width 0.25) (layer "F.Cu") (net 31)))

